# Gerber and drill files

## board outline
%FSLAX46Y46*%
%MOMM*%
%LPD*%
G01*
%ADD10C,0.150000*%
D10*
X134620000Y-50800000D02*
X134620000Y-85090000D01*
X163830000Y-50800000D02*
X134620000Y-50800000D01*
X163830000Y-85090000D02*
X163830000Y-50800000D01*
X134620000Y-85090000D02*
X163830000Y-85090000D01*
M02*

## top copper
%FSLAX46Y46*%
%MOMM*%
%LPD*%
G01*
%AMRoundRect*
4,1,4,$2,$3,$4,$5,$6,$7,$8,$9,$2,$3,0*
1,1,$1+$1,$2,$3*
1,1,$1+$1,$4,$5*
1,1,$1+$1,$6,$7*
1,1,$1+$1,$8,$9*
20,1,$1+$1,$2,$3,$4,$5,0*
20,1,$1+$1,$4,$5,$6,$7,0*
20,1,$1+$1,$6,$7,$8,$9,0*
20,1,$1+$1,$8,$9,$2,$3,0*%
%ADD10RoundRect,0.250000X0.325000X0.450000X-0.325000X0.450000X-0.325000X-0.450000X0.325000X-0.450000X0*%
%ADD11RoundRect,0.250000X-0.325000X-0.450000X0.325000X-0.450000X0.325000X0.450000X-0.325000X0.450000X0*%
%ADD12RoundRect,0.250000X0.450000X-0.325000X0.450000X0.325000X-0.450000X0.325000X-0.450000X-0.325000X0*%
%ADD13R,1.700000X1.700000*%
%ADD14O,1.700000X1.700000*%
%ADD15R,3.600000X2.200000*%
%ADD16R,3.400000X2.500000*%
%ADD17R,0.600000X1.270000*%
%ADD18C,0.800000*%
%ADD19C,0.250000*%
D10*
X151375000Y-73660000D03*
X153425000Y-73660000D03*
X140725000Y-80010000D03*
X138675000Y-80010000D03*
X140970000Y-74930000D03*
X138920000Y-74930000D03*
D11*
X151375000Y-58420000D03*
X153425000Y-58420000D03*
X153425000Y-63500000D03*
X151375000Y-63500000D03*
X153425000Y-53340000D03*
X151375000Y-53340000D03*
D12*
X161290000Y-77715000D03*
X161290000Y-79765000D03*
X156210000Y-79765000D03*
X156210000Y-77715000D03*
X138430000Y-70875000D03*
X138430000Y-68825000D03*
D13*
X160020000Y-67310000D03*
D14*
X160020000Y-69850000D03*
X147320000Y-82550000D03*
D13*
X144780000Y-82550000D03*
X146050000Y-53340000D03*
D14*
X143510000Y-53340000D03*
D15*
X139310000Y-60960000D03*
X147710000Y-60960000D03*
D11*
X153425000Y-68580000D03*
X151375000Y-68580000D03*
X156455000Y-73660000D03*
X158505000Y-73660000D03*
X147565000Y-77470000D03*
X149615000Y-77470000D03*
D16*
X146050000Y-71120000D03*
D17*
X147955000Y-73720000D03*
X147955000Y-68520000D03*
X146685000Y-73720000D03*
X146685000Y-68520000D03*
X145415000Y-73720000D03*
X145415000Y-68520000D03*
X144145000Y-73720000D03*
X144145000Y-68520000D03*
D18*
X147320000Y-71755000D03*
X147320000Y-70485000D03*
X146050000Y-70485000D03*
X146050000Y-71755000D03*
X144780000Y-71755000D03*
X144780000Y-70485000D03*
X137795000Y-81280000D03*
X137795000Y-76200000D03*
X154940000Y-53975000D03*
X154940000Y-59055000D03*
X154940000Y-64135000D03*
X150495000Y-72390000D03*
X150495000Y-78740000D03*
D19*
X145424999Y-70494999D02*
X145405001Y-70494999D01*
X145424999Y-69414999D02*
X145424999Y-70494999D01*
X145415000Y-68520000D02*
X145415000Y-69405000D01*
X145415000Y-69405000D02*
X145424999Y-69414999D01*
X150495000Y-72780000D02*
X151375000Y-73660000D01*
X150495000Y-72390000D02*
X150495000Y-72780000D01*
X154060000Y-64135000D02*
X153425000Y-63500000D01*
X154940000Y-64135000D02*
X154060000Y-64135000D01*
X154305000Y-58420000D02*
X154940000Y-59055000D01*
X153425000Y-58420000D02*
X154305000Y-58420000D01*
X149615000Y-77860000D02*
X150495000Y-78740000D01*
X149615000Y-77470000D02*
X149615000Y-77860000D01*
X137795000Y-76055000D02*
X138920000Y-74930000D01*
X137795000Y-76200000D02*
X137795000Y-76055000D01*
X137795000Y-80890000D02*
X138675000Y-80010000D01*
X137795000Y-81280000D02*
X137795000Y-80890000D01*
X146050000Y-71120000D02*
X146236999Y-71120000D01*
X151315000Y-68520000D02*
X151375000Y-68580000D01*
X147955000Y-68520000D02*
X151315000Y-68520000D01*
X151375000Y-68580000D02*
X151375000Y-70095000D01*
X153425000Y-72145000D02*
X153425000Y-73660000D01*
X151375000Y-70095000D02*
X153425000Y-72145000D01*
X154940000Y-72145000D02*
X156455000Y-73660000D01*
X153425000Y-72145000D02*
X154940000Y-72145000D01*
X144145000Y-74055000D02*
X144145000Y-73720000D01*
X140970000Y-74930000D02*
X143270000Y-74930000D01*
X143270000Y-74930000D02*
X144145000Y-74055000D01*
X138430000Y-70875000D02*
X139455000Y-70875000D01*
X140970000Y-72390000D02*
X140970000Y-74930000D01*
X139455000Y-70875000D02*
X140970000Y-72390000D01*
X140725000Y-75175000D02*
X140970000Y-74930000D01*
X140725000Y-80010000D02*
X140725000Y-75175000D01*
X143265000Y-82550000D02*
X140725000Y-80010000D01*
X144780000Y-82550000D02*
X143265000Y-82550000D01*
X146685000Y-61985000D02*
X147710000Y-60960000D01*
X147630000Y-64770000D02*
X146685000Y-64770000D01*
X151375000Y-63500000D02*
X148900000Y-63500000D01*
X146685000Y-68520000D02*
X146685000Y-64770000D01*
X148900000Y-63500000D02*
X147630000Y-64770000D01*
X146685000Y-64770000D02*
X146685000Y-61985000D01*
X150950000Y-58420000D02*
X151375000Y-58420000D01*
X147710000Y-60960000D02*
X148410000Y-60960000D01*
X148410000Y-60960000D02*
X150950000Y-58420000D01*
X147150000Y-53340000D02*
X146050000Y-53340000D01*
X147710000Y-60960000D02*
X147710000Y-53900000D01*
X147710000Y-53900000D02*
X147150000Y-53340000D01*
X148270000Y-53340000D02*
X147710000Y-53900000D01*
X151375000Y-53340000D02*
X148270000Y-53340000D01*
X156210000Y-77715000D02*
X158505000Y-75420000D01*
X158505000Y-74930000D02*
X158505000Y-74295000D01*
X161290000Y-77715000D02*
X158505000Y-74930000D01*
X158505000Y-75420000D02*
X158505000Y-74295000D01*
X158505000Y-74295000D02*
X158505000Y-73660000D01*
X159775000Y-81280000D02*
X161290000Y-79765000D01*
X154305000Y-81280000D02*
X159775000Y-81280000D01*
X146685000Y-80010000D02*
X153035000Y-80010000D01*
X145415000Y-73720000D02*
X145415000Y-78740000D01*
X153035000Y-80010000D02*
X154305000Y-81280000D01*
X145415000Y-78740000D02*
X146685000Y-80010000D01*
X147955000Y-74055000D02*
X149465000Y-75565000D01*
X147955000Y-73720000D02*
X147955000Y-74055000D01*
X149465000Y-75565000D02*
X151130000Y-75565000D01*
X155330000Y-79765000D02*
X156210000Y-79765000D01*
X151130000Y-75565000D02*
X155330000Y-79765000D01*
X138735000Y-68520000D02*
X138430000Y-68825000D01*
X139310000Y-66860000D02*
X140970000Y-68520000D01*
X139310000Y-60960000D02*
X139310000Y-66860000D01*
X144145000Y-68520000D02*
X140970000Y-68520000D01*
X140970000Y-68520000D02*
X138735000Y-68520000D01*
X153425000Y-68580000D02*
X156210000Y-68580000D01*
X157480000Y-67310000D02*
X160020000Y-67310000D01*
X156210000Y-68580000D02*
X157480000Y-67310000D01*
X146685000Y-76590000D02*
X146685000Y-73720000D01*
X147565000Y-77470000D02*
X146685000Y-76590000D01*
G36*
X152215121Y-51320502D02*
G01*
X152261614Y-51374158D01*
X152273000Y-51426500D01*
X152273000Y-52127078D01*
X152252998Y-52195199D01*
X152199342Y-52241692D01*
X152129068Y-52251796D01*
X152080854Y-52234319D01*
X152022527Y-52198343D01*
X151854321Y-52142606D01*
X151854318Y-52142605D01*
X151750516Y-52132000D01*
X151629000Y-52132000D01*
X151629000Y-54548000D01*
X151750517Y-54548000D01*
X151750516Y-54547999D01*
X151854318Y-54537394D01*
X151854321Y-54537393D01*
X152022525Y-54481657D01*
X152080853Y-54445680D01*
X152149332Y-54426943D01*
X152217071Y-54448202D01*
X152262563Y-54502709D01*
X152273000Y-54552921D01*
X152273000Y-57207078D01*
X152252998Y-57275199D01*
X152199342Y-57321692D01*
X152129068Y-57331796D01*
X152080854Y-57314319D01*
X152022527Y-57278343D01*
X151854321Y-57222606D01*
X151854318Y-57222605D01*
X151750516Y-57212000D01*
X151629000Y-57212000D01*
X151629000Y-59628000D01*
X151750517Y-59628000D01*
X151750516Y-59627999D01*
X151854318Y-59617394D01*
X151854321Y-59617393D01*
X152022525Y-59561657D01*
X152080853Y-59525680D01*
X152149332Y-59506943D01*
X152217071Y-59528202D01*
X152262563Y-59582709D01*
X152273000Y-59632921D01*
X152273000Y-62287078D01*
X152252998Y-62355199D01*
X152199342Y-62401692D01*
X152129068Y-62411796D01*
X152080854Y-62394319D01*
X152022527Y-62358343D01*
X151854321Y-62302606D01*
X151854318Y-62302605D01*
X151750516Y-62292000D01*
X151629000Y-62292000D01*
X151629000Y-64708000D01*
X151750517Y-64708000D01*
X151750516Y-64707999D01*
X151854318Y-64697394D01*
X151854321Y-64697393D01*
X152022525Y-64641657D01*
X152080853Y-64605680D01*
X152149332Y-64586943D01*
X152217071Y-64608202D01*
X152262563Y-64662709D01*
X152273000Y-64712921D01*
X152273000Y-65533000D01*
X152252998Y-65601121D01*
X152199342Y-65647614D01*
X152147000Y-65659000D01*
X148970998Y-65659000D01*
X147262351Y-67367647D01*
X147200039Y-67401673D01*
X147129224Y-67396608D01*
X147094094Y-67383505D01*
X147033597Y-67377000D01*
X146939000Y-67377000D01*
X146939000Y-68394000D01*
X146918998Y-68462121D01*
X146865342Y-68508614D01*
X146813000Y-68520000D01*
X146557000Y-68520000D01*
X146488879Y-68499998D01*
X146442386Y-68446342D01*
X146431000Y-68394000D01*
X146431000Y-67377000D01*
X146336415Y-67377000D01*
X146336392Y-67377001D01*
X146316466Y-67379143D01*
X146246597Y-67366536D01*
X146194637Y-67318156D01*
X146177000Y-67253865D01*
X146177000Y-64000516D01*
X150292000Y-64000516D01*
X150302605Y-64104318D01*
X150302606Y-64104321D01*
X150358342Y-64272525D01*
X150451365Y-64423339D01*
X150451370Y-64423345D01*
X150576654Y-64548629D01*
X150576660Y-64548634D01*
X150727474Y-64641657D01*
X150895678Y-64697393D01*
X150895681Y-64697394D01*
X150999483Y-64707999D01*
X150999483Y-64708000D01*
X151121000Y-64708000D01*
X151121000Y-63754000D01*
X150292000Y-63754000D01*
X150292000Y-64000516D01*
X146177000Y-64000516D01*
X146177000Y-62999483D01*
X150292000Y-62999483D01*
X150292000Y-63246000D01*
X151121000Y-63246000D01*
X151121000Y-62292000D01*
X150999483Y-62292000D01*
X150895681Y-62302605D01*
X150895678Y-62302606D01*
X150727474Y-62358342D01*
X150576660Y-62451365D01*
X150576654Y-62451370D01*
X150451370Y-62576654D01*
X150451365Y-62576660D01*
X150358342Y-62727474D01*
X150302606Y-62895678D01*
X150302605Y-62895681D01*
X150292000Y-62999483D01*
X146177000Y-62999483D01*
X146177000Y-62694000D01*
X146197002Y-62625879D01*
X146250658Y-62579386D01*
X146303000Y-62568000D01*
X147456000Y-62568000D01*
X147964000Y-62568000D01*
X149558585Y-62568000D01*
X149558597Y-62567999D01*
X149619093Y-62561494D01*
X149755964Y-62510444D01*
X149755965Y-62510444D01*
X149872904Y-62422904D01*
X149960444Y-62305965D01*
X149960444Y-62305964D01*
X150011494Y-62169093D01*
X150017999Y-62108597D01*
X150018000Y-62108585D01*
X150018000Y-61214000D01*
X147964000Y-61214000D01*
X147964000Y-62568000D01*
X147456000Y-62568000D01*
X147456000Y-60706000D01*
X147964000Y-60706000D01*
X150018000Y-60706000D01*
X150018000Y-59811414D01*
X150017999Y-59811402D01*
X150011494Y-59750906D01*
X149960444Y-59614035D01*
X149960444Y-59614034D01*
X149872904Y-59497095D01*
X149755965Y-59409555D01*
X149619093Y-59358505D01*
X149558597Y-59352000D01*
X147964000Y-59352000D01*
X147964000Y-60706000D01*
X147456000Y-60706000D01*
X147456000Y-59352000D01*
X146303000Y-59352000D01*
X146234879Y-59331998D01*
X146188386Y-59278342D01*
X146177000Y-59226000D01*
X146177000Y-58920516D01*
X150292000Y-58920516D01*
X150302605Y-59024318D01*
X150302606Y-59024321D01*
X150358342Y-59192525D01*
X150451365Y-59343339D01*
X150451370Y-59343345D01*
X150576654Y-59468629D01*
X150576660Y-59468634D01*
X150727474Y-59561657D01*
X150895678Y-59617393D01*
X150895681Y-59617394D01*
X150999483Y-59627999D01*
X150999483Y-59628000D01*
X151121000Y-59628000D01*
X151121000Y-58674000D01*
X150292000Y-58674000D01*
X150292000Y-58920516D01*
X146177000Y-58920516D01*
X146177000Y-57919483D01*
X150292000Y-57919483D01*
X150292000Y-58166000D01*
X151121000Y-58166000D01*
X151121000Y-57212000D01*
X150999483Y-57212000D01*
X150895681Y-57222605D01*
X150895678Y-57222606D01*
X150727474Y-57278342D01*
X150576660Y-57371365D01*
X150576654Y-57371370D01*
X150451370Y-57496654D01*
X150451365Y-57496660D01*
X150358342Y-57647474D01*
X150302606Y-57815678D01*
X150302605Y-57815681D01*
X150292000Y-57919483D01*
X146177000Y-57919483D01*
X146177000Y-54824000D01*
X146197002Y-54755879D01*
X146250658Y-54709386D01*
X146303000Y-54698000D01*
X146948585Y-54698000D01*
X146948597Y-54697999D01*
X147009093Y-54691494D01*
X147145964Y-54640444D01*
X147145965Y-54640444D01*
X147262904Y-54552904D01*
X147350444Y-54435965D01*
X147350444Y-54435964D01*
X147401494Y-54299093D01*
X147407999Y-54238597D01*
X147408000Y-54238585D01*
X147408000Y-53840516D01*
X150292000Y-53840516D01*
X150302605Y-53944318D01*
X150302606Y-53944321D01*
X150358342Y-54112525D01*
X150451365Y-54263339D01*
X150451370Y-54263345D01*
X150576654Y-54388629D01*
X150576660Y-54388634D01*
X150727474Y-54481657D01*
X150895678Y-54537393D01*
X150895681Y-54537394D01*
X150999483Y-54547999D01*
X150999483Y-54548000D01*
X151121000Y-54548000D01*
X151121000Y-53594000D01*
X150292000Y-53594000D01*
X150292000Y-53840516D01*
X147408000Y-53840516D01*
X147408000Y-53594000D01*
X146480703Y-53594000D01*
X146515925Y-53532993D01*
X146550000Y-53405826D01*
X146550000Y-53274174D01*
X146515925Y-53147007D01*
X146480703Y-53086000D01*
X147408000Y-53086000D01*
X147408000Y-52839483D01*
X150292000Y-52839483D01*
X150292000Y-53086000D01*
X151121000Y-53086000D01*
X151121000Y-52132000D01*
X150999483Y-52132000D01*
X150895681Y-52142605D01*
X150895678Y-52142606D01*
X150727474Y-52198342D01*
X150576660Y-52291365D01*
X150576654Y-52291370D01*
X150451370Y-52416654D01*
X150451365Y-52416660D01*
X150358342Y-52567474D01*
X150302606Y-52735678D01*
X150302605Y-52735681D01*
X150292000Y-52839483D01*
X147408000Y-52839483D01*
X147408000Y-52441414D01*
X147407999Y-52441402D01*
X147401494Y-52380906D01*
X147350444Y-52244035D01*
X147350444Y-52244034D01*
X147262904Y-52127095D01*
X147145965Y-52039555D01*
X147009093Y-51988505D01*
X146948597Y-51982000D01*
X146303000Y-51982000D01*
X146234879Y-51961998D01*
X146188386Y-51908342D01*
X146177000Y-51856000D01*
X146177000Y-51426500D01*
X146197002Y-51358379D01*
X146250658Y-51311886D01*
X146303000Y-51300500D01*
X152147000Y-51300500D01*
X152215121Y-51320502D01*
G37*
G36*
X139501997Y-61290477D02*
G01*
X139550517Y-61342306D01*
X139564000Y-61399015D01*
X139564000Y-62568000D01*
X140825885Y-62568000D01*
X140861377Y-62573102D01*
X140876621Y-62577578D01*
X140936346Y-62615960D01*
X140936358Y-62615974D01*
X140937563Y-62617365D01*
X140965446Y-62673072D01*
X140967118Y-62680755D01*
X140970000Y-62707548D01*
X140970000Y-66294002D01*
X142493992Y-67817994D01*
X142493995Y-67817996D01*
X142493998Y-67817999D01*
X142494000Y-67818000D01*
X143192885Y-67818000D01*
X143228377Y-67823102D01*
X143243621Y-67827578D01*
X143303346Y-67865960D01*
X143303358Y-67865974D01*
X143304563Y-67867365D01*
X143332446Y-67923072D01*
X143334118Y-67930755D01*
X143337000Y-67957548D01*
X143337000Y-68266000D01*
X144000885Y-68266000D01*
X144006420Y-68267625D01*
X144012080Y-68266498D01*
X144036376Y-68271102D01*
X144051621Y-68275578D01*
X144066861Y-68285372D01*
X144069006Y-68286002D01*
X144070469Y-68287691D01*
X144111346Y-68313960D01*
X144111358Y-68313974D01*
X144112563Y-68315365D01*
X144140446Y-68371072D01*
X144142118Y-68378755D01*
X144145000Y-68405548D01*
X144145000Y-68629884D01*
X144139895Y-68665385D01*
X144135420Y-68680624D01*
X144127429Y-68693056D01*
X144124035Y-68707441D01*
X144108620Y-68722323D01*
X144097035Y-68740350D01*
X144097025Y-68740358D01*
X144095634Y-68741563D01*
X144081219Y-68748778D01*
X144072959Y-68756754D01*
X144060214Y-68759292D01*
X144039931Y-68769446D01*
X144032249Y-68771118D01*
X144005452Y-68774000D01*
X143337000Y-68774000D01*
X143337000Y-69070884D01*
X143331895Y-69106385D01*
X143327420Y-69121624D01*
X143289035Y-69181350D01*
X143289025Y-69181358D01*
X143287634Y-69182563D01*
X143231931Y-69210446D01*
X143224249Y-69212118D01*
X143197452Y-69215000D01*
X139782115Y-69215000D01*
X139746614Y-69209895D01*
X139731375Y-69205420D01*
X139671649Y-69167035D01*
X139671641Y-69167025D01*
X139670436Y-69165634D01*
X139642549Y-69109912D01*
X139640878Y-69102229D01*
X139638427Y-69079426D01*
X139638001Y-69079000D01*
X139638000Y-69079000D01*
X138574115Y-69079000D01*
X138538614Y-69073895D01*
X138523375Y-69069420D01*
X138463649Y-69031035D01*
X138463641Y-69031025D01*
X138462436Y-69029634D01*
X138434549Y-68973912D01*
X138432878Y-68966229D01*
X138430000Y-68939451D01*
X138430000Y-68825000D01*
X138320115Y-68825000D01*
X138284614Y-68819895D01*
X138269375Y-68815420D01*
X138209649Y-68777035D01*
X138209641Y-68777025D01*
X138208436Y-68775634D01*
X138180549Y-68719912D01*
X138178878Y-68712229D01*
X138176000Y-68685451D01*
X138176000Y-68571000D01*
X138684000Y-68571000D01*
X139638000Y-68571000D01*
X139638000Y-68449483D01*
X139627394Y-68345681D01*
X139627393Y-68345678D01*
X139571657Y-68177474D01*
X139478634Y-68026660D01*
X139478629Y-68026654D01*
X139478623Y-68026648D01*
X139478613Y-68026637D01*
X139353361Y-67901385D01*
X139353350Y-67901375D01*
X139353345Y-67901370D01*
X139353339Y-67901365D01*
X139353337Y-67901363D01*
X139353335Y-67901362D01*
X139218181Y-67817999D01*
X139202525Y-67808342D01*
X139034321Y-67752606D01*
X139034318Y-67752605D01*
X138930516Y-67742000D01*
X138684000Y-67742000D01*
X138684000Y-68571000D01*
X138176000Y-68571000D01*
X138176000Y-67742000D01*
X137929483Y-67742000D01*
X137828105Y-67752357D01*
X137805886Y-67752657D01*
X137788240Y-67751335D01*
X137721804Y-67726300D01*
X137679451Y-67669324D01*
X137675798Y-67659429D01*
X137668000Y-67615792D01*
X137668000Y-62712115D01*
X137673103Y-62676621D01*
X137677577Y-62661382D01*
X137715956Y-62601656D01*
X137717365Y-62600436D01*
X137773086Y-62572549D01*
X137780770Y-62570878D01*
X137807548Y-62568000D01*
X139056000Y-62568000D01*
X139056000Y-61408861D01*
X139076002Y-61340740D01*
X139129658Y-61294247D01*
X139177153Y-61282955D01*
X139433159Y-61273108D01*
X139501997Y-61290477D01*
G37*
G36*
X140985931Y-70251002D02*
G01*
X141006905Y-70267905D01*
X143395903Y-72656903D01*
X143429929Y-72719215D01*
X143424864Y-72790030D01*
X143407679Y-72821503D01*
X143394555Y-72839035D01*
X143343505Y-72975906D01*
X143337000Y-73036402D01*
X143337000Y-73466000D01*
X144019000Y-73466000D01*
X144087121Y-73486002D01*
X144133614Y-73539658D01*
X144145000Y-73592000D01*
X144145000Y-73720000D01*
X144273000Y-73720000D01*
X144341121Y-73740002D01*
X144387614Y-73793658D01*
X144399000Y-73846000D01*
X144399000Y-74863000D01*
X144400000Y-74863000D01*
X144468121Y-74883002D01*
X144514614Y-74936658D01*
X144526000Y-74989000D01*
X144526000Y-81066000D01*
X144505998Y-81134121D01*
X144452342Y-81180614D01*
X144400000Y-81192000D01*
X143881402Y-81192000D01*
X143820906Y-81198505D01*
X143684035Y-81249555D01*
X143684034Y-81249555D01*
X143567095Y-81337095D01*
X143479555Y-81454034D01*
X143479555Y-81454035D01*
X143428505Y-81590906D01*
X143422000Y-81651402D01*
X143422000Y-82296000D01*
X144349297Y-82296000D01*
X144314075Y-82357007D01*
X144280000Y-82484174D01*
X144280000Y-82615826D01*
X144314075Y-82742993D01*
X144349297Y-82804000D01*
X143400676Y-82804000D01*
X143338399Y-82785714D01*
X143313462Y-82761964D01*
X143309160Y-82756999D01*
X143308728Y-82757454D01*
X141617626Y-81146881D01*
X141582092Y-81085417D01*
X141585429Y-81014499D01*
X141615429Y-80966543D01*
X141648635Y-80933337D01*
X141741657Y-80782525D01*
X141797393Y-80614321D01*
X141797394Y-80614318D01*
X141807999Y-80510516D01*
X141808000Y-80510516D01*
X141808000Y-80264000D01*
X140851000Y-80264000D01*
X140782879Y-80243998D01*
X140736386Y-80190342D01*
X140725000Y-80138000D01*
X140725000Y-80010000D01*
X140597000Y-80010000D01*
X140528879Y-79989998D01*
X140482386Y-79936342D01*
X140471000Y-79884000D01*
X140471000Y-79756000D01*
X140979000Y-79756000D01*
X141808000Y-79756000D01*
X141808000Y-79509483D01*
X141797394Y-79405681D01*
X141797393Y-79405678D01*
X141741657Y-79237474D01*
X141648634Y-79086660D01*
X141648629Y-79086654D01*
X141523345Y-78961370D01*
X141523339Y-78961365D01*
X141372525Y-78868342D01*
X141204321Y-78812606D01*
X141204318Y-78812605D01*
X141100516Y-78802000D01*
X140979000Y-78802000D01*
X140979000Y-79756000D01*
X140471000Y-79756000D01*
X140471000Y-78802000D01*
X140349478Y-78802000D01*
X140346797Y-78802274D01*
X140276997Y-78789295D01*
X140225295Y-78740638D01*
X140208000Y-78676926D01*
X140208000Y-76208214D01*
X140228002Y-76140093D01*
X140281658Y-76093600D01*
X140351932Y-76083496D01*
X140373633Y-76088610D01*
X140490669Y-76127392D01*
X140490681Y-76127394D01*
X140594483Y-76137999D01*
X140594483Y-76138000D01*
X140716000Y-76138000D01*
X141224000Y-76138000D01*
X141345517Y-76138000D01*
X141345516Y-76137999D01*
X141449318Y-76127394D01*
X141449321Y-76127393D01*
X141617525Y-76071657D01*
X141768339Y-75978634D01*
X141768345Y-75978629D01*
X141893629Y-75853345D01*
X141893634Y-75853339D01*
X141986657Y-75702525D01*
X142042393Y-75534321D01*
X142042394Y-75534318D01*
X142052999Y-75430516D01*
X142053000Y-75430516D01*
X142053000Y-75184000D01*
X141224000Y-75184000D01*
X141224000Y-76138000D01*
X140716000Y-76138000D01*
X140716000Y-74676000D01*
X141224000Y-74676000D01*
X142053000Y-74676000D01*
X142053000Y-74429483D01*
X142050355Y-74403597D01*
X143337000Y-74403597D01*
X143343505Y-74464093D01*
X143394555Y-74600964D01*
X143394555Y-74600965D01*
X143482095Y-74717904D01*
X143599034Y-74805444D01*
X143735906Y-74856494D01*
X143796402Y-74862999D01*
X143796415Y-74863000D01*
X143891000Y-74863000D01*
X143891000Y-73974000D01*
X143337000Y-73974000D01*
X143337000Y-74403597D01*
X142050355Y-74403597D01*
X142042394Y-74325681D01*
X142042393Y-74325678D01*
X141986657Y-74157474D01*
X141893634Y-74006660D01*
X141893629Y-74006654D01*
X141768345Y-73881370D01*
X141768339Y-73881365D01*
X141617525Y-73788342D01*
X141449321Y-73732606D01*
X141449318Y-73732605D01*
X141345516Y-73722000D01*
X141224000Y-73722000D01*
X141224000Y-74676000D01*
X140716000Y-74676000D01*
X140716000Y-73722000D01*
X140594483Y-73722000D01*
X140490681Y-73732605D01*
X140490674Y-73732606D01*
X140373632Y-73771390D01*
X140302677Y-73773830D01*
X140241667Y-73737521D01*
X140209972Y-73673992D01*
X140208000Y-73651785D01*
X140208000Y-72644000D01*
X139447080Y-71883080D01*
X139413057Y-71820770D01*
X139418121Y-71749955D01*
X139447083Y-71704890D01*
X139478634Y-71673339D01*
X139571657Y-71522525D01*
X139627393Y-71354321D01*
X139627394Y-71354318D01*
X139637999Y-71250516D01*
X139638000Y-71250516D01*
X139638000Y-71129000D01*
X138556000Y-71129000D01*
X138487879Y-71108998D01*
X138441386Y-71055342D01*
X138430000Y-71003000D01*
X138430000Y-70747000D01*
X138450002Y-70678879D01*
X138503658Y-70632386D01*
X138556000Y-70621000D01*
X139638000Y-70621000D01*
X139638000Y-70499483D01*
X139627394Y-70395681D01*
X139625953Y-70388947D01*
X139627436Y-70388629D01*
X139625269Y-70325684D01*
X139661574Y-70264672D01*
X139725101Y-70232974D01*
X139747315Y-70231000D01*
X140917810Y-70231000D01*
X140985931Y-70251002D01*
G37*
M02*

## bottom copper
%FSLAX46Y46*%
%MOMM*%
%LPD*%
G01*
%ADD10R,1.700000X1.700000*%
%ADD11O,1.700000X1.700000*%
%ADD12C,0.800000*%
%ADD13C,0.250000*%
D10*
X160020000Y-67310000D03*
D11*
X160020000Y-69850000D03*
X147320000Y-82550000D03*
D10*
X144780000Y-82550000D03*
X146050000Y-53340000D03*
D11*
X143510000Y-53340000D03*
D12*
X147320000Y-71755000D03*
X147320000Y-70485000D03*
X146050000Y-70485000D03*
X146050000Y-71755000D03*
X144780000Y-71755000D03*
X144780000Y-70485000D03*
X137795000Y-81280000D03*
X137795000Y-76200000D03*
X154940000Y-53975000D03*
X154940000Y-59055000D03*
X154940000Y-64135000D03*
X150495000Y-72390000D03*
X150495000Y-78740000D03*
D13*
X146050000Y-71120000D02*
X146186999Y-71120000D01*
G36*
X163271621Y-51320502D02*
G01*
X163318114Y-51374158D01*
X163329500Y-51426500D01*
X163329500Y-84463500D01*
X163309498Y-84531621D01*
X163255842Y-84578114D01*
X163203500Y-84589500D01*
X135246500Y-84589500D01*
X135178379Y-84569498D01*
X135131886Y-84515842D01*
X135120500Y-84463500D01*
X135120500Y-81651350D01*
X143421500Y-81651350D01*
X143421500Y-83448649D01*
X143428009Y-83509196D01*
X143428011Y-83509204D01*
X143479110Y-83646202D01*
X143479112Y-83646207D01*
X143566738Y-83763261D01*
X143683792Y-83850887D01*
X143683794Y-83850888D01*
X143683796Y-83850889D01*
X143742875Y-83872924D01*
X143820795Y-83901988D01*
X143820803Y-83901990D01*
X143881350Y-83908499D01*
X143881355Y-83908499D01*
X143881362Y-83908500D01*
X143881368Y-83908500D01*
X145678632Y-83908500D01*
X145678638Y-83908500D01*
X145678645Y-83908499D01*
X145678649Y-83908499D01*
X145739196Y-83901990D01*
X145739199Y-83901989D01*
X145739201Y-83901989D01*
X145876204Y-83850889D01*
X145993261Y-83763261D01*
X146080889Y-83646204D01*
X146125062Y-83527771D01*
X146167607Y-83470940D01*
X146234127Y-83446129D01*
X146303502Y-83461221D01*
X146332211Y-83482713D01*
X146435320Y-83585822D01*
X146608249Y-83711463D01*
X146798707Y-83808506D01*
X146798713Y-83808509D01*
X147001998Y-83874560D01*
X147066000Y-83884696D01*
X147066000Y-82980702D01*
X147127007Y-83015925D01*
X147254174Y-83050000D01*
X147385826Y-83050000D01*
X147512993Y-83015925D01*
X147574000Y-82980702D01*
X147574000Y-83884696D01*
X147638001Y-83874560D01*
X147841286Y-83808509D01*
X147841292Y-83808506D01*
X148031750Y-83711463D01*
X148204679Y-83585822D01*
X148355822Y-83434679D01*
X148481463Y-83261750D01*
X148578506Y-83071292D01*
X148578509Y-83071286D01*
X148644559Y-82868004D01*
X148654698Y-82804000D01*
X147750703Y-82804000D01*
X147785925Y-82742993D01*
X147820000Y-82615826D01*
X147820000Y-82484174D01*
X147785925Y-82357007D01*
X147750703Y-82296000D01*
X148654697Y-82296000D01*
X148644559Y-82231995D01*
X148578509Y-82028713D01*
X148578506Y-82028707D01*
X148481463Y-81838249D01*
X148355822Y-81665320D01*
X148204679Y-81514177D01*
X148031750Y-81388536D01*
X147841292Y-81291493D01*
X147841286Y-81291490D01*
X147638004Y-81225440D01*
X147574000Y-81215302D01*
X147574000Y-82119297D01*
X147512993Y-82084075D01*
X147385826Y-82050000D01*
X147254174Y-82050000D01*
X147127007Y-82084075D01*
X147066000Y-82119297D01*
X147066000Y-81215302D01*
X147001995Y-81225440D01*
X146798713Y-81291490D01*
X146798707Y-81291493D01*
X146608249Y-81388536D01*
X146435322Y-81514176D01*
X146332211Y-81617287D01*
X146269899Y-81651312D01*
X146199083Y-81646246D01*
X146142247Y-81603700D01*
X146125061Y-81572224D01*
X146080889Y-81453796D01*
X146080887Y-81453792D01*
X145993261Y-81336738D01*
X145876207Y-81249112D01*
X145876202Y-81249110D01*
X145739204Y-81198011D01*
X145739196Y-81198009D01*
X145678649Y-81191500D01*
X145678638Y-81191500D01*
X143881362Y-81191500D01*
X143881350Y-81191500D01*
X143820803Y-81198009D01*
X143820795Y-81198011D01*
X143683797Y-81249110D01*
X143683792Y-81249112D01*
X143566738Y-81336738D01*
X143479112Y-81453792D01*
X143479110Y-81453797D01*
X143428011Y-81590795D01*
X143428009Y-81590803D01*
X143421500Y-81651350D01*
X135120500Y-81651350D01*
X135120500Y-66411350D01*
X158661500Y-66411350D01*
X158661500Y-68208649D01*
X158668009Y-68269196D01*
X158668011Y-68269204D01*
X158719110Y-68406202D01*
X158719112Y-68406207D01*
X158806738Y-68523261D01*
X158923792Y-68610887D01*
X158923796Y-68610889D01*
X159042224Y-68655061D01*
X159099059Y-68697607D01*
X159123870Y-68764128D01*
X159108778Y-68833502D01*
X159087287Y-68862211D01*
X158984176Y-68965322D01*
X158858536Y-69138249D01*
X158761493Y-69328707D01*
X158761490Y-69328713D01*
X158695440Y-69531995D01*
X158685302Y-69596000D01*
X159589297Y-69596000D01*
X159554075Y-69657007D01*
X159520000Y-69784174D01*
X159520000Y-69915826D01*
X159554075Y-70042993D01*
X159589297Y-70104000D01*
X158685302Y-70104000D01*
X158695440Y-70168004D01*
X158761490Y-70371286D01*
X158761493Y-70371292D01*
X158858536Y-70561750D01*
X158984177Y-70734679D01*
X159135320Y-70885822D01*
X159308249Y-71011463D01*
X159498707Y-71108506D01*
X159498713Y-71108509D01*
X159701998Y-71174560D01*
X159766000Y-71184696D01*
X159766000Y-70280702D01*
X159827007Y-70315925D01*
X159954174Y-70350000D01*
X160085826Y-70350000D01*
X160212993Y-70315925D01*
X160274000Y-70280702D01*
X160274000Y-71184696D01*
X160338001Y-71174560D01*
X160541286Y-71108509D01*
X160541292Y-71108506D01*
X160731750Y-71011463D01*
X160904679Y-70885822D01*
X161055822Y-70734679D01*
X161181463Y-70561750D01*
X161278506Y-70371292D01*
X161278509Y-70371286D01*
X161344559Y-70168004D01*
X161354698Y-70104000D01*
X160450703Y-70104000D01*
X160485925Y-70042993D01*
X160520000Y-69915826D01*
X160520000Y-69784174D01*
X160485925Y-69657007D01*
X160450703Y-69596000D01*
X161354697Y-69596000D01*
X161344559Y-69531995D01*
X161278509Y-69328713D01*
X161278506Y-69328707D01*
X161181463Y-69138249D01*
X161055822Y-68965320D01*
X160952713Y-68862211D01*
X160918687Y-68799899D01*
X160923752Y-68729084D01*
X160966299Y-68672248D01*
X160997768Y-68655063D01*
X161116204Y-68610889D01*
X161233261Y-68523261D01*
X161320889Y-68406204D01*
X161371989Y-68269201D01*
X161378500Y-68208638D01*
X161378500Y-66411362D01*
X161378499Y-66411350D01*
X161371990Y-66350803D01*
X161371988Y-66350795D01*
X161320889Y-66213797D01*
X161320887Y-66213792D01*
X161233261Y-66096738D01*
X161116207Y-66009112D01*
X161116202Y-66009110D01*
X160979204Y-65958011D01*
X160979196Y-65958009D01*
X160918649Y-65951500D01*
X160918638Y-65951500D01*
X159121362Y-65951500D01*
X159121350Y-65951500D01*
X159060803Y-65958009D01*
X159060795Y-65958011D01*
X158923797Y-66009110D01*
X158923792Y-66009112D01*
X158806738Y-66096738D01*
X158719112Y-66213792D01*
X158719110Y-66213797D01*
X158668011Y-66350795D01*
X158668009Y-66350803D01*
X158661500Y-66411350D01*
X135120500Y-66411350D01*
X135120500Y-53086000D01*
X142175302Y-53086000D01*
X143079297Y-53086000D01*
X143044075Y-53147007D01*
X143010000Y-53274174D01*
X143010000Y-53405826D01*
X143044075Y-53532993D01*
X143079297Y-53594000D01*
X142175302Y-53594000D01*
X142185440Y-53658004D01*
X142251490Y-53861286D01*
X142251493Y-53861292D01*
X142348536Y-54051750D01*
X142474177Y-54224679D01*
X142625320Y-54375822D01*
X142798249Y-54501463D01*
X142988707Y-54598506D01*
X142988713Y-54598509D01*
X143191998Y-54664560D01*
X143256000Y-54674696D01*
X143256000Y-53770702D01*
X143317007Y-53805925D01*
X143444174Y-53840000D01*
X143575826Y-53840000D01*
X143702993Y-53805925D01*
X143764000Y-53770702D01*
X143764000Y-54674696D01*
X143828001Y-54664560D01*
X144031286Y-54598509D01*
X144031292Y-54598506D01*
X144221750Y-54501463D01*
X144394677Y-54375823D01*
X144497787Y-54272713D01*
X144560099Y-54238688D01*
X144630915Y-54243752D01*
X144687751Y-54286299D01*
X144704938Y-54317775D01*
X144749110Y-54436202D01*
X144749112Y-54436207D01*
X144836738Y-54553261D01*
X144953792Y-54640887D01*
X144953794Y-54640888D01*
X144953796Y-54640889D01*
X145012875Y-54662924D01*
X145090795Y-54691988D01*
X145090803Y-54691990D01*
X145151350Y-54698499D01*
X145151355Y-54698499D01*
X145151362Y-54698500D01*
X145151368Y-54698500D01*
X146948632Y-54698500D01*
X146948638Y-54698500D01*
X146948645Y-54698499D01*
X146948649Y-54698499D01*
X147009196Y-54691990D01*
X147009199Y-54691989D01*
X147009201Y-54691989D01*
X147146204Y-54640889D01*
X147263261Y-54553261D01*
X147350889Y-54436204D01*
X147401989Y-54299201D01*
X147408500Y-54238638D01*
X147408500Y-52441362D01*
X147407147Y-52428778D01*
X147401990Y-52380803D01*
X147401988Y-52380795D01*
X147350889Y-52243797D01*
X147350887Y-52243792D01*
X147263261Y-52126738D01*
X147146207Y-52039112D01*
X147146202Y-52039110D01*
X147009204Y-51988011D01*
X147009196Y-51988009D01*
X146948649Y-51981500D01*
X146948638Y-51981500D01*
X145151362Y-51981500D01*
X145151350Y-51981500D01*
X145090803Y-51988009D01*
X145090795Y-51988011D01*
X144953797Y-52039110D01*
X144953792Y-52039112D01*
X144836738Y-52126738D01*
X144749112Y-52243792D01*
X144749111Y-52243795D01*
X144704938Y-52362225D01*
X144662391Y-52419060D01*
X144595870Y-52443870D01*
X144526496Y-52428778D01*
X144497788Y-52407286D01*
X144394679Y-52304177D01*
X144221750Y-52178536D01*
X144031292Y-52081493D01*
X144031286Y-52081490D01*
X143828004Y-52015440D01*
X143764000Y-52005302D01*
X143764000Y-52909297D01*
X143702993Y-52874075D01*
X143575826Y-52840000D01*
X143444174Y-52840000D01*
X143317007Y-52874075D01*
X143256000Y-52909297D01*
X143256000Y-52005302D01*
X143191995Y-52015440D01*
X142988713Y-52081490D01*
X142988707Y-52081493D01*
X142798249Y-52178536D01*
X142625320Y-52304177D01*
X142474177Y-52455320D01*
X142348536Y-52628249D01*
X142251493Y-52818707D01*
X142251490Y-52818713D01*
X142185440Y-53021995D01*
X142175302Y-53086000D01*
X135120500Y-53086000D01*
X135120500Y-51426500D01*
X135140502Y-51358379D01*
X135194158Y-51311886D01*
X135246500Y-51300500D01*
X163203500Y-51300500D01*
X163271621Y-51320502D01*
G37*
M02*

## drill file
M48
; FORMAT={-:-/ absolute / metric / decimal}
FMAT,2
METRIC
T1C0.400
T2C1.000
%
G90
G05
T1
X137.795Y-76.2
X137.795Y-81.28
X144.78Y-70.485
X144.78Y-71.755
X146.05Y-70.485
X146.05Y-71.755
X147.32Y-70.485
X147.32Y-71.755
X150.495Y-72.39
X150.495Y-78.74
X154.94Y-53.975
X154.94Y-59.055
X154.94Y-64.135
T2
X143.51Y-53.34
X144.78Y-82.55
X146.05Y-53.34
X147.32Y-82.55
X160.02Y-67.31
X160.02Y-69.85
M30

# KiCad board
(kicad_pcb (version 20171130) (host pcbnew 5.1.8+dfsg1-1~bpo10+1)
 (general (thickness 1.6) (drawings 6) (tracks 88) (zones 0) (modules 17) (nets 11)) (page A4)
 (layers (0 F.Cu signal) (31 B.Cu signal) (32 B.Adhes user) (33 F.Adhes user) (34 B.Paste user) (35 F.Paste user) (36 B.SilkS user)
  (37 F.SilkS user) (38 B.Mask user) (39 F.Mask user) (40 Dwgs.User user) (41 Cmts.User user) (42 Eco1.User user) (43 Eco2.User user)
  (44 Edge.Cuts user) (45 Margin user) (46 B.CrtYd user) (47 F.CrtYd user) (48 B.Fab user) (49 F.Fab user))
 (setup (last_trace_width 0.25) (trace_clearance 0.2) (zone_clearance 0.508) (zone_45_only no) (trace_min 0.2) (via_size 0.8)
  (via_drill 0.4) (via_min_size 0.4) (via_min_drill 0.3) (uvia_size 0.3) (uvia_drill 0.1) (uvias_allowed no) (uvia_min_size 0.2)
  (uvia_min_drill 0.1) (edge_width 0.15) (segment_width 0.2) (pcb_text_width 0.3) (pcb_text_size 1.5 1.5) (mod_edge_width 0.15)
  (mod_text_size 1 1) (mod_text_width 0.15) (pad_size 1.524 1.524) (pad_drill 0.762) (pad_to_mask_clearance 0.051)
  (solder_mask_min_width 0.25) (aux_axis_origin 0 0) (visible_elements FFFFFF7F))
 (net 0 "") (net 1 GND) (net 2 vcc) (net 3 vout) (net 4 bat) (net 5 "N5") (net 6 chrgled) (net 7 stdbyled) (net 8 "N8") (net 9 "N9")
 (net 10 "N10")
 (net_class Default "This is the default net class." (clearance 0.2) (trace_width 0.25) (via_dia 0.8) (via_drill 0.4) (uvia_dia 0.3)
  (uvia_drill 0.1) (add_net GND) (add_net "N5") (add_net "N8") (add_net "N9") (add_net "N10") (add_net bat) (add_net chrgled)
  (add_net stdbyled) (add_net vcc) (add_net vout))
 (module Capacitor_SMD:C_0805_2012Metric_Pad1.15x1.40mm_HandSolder (layer F.Cu) (at 152.4 73.66 180)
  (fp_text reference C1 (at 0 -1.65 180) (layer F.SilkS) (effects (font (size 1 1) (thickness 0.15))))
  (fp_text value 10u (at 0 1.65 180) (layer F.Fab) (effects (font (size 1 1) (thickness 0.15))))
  (pad 2 smd roundrect (at 1.025 0 180) (size 1.15 1.4) (layers F.Cu F.Paste F.Mask) (roundrect_rratio 0.217391) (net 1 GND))
  (pad 1 smd roundrect (at -1.025 0 180) (size 1.15 1.4) (layers F.Cu F.Paste F.Mask) (roundrect_rratio 0.217391) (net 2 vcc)))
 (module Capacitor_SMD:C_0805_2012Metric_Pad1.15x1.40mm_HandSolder (layer F.Cu) (at 139.7 80.01 180)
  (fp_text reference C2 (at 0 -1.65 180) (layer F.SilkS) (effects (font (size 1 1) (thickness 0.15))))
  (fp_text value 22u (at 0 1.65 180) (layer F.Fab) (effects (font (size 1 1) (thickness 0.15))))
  (pad 1 smd roundrect (at -1.025 0 180) (size 1.15 1.4) (layers F.Cu F.Paste F.Mask) (roundrect_rratio 0.217391) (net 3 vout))
  (pad 2 smd roundrect (at 1.025 0 180) (size 1.15 1.4) (layers F.Cu F.Paste F.Mask) (roundrect_rratio 0.217391) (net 1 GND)))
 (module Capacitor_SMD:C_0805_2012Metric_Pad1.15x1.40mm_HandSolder (layer F.Cu) (at 139.945 74.93 180)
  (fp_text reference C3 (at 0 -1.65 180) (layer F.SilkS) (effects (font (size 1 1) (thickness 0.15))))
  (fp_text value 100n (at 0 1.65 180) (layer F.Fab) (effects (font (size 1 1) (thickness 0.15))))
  (pad 1 smd roundrect (at -1.025 0 180) (size 1.15 1.4) (layers F.Cu F.Paste F.Mask) (roundrect_rratio 0.217391) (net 3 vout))
  (pad 2 smd roundrect (at 1.025 0 180) (size 1.15 1.4) (layers F.Cu F.Paste F.Mask) (roundrect_rratio 0.217391) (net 1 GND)))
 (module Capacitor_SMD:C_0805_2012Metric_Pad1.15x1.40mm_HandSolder (layer F.Cu) (at 152.4 58.42)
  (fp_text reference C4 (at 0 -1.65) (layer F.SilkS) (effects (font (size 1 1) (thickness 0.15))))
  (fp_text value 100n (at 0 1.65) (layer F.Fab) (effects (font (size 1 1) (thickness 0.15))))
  (pad 1 smd roundrect (at -1.025 0) (size 1.15 1.4) (layers F.Cu F.Paste F.Mask) (roundrect_rratio 0.217391) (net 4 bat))
  (pad 2 smd roundrect (at 1.025 0) (size 1.15 1.4) (layers F.Cu F.Paste F.Mask) (roundrect_rratio 0.217391) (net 1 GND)))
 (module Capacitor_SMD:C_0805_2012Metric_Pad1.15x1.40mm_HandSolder (layer F.Cu) (at 152.4 63.5)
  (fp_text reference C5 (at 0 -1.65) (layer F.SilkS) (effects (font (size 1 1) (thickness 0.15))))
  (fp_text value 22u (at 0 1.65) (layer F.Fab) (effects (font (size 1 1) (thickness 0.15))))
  (pad 2 smd roundrect (at 1.025 0) (size 1.15 1.4) (layers F.Cu F.Paste F.Mask) (roundrect_rratio 0.217391) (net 1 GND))
  (pad 1 smd roundrect (at -1.025 0) (size 1.15 1.4) (layers F.Cu F.Paste F.Mask) (roundrect_rratio 0.217391) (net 4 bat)))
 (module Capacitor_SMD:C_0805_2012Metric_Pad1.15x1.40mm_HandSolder (layer F.Cu) (at 152.4 53.34)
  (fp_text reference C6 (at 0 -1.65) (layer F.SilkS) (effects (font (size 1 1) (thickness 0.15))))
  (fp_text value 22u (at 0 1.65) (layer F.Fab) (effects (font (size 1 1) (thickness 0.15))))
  (pad 2 smd roundrect (at 1.025 0) (size 1.15 1.4) (layers F.Cu F.Paste F.Mask) (roundrect_rratio 0.217391) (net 1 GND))
  (pad 1 smd roundrect (at -1.025 0) (size 1.15 1.4) (layers F.Cu F.Paste F.Mask) (roundrect_rratio 0.217391) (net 4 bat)))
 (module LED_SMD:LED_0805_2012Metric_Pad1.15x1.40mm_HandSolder (layer F.Cu) (at 161.29 78.74 90)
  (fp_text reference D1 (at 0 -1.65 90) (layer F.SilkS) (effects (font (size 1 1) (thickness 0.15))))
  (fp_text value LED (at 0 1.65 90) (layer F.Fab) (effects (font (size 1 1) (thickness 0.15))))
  (pad 2 smd roundrect (at 1.025 0 90) (size 1.15 1.4) (layers F.Cu F.Paste F.Mask) (roundrect_rratio 0.217391) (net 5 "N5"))
  (pad 1 smd roundrect (at -1.025 0 90) (size 1.15 1.4) (layers F.Cu F.Paste F.Mask) (roundrect_rratio 0.217391) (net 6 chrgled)))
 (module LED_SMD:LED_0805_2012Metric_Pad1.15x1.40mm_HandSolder (layer F.Cu) (at 156.21 78.74 90)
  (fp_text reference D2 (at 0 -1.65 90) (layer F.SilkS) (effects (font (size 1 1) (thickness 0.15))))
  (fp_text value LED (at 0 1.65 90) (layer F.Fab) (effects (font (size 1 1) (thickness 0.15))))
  (pad 1 smd roundrect (at -1.025 0 90) (size 1.15 1.4) (layers F.Cu F.Paste F.Mask) (roundrect_rratio 0.217391) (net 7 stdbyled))
  (pad 2 smd roundrect (at 1.025 0 90) (size 1.15 1.4) (layers F.Cu F.Paste F.Mask) (roundrect_rratio 0.217391) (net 5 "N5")))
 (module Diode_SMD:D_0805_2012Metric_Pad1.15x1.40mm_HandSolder (layer F.Cu) (at 138.43 69.85 90)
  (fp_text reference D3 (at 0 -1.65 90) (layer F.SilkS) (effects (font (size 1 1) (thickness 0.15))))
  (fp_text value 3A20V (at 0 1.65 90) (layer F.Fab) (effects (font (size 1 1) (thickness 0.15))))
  (pad 1 smd roundrect (at -1.025 0 90) (size 1.15 1.4) (layers F.Cu F.Paste F.Mask) (roundrect_rratio 0.217391) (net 3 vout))
  (pad 2 smd roundrect (at 1.025 0 90) (size 1.15 1.4) (layers F.Cu F.Paste F.Mask) (roundrect_rratio 0.217391) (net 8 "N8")))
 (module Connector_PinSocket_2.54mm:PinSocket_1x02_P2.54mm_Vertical (layer F.Cu) (at 160.02 67.31)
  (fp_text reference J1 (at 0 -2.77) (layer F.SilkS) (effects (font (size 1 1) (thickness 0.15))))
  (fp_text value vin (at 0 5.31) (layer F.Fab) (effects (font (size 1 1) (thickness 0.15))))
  (pad 1 thru_hole rect (at 0 0) (size 1.7 1.7) (drill 1) (layers *.Cu *.Mask) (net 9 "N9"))
  (pad 2 thru_hole oval (at 0 2.54) (size 1.7 1.7) (drill 1) (layers *.Cu *.Mask) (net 1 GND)))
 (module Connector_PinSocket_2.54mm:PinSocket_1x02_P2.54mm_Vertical (layer F.Cu) (at 144.78 82.55 90)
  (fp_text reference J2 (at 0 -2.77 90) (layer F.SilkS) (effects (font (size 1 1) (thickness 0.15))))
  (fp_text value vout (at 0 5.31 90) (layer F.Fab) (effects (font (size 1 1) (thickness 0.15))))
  (pad 2 thru_hole oval (at 0 2.54 90) (size 1.7 1.7) (drill 1) (layers *.Cu *.Mask) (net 1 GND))
  (pad 1 thru_hole rect (at 0 0 90) (size 1.7 1.7) (drill 1) (layers *.Cu *.Mask) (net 3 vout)))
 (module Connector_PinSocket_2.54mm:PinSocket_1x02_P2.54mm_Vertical (layer F.Cu) (at 146.05 53.34 270)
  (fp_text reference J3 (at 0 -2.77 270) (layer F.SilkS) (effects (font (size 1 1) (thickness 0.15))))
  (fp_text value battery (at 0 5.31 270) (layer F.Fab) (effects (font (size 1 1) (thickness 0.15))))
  (pad 1 thru_hole rect (at 0 0 270) (size 1.7 1.7) (drill 1) (layers *.Cu *.Mask) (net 4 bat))
  (pad 2 thru_hole oval (at 0 2.54 270) (size 1.7 1.7) (drill 1) (layers *.Cu *.Mask) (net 1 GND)))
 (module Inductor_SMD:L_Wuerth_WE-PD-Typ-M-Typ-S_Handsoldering (layer F.Cu) (at 143.51 60.96)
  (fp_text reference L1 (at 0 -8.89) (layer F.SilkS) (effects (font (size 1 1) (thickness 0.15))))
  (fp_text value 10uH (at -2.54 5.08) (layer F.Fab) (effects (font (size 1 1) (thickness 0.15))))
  (pad 1 smd rect (at -4.2 0) (size 3.6 2.2) (layers F.Cu F.Paste F.Mask) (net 8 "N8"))
  (pad 2 smd rect (at 4.2 0) (size 3.6 2.2) (layers F.Cu F.Paste F.Mask) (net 4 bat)))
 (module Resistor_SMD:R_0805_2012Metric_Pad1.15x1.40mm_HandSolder (layer F.Cu) (at 152.4 68.58)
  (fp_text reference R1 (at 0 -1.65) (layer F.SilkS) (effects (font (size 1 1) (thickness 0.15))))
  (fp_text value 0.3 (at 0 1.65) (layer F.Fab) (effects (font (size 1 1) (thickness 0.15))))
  (pad 2 smd roundrect (at 1.025 0) (size 1.15 1.4) (layers F.Cu F.Paste F.Mask) (roundrect_rratio 0.217391) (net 9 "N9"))
  (pad 1 smd roundrect (at -1.025 0) (size 1.15 1.4) (layers F.Cu F.Paste F.Mask) (roundrect_rratio 0.217391) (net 2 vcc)))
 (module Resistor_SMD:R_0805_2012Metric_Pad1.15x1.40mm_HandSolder (layer F.Cu) (at 157.48 73.66)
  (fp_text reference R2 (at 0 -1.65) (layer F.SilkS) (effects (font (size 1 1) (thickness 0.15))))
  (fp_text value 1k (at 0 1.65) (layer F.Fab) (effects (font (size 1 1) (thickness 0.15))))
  (pad 1 smd roundrect (at -1.025 0) (size 1.15 1.4) (layers F.Cu F.Paste F.Mask) (roundrect_rratio 0.217391) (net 2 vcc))
  (pad 2 smd roundrect (at 1.025 0) (size 1.15 1.4) (layers F.Cu F.Paste F.Mask) (roundrect_rratio 0.217391) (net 5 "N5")))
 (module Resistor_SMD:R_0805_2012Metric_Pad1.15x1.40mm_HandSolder (layer F.Cu) (at 148.59 77.47)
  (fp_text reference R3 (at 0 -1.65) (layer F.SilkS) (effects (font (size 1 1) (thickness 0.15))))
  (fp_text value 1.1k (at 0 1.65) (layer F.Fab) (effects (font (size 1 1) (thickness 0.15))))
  (pad 1 smd roundrect (at -1.025 0) (size 1.15 1.4) (layers F.Cu F.Paste F.Mask) (roundrect_rratio 0.217391) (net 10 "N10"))
  (pad 2 smd roundrect (at 1.025 0) (size 1.15 1.4) (layers F.Cu F.Paste F.Mask) (roundrect_rratio 0.217391) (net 1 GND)))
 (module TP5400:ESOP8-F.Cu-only (layer F.Cu) (at 146.05 71.12)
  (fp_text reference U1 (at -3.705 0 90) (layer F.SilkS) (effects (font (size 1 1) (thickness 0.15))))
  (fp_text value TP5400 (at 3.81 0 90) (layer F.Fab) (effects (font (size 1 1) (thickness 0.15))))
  (pad 9 smd rect (at 0 0) (size 3.4 2.5) (layers F.Cu F.Paste F.Mask) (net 1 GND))
  (pad 4 smd rect (at 1.905 2.6) (size 0.6 1.27) (layers F.Cu F.Paste F.Mask) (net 7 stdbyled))
  (pad 5 smd rect (at 1.905 -2.6) (size 0.6 1.27) (layers F.Cu F.Paste F.Mask) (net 2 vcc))
  (pad 3 smd rect (at 0.635 2.6) (size 0.6 1.27) (layers F.Cu F.Paste F.Mask) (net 10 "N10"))
  (pad 6 smd rect (at 0.635 -2.6) (size 0.6 1.27) (layers F.Cu F.Paste F.Mask) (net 4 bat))
  (pad 2 smd rect (at -0.635 2.6) (size 0.6 1.27) (layers F.Cu F.Paste F.Mask) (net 6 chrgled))
  (pad 7 smd rect (at -0.635 -2.6) (size 0.6 1.27) (layers F.Cu F.Paste F.Mask) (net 1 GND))
  (pad 1 smd rect (at -1.905 2.6) (size 0.6 1.27) (layers F.Cu F.Paste F.Mask) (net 3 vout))
  (pad 8 smd rect (at -1.905 -2.6) (size 0.6 1.27) (layers F.Cu F.Paste F.Mask) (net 8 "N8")))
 (gr_line (start 134.62 50.8) (end 134.62 85.09) (layer Edge.Cuts) (width 0.15))
 (gr_line (start 163.83 50.8) (end 134.62 50.8) (layer Edge.Cuts) (width 0.15))
 (gr_line (start 163.83 85.09) (end 163.83 50.8) (layer Edge.Cuts) (width 0.15))
 (gr_line (start 134.62 85.09) (end 163.83 85.09) (layer Edge.Cuts) (width 0.15))
 (via (at 147.32 71.755) (size 0.8) (drill 0.4) (layers F.Cu B.Cu) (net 1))
 (via (at 147.32 70.485) (size 0.8) (drill 0.4) (layers F.Cu B.Cu) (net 1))
 (via (at 146.05 70.485) (size 0.8) (drill 0.4) (layers F.Cu B.Cu) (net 1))
 (via (at 146.05 71.755) (size 0.8) (drill 0.4) (layers F.Cu B.Cu) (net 1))
 (via (at 144.78 71.755) (size 0.8) (drill 0.4) (layers F.Cu B.Cu) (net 1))
 (via (at 144.78 70.485) (size 0.8) (drill 0.4) (layers F.Cu B.Cu) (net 1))
 (segment (start 145.424999 70.494999) (end 145.405001 70.494999) (width 0.25) (layer F.Cu) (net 1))
 (segment (start 145.424999 69.414999) (end 145.424999 70.494999) (width 0.25) (layer F.Cu) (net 1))
 (segment (start 145.415 68.52) (end 145.415 69.405) (width 0.25) (layer F.Cu) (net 1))
 (segment (start 145.415 69.405) (end 145.424999 69.414999) (width 0.25) (layer F.Cu) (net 1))
 (via (at 137.795 81.28) (size 0.8) (drill 0.4) (layers F.Cu B.Cu) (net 1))
 (via (at 137.795 76.2) (size 0.8) (drill 0.4) (layers F.Cu B.Cu) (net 1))
 (via (at 154.94 53.975) (size 0.8) (drill 0.4) (layers F.Cu B.Cu) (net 1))
 (via (at 154.94 59.055) (size 0.8) (drill 0.4) (layers F.Cu B.Cu) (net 1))
 (via (at 154.94 64.135) (size 0.8) (drill 0.4) (layers F.Cu B.Cu) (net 1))
 (via (at 150.495 72.39) (size 0.8) (drill 0.4) (layers F.Cu B.Cu) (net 1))
 (via (at 150.495 78.74) (size 0.8) (drill 0.4) (layers F.Cu B.Cu) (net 1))
 (segment (start 150.495 72.78) (end 151.375 73.66) (width 0.25) (layer F.Cu) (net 1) (status 20))
 (segment (start 150.495 72.39) (end 150.495 72.78) (width 0.25) (layer F.Cu) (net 1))
 (segment (start 154.06 64.135) (end 153.425 63.5) (width 0.25) (layer F.Cu) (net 1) (status 20))
 (segment (start 154.94 64.135) (end 154.06 64.135) (width 0.25) (layer F.Cu) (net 1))
 (segment (start 154.305 58.42) (end 154.94 59.055) (width 0.25) (layer F.Cu) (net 1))
 (segment (start 153.425 58.42) (end 154.305 58.42) (width 0.25) (layer F.Cu) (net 1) (status 10))
 (segment (start 149.615 77.86) (end 150.495 78.74) (width 0.25) (layer F.Cu) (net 1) (status 10))
 (segment (start 149.615 77.47) (end 149.615 77.86) (width 0.25) (layer F.Cu) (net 1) (status 30))
 (segment (start 137.795 76.055) (end 138.92 74.93) (width 0.25) (layer F.Cu) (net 1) (status 20))
 (segment (start 137.795 76.2) (end 137.795 76.055) (width 0.25) (layer F.Cu) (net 1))
 (segment (start 137.795 80.89) (end 138.675 80.01) (width 0.25) (layer F.Cu) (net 1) (status 20))
 (segment (start 137.795 81.28) (end 137.795 80.89) (width 0.25) (layer F.Cu) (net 1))
 (segment (start 146.05 71.12) (end 146.186999 71.12) (width 0.25) (layer B.Cu) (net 1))
 (segment (start 146.05 71.12) (end 146.236999 71.12) (width 0.25) (layer F.Cu) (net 1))
 (segment (start 151.315 68.52) (end 151.375 68.58) (width 0.25) (layer F.Cu) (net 2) (status 30))
 (segment (start 147.955 68.52) (end 151.315 68.52) (width 0.25) (layer F.Cu) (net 2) (status 20))
 (segment (start 151.375 68.58) (end 151.375 70.095) (width 0.25) (layer F.Cu) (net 2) (status 10))
 (segment (start 153.425 72.145) (end 153.425 73.66) (width 0.25) (layer F.Cu) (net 2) (status 20))
 (segment (start 151.375 70.095) (end 153.425 72.145) (width 0.25) (layer F.Cu) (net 2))
 (segment (start 154.94 72.145) (end 156.455 73.66) (width 0.25) (layer F.Cu) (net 2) (status 20))
 (segment (start 153.425 72.145) (end 154.94 72.145) (width 0.25) (layer F.Cu) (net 2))
 (segment (start 144.145 74.055) (end 144.145 73.72) (width 0.25) (layer F.Cu) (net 3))
 (segment (start 140.97 74.93) (end 143.27 74.93) (width 0.25) (layer F.Cu) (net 3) (status 10))
 (segment (start 143.27 74.93) (end 144.145 74.055) (width 0.25) (layer F.Cu) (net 3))
 (segment (start 138.43 70.875) (end 139.455 70.875) (width 0.25) (layer F.Cu) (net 3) (status 10))
 (segment (start 140.97 72.39) (end 140.97 74.93) (width 0.25) (layer F.Cu) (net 3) (status 20))
 (segment (start 139.455 70.875) (end 140.97 72.39) (width 0.25) (layer F.Cu) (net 3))
 (segment (start 140.725 75.175) (end 140.97 74.93) (width 0.25) (layer F.Cu) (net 3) (status 30))
 (segment (start 140.725 80.01) (end 140.725 75.175) (width 0.25) (layer F.Cu) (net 3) (status 30))
 (segment (start 143.265 82.55) (end 140.725 80.01) (width 0.25) (layer F.Cu) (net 3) (status 20))
 (segment (start 144.78 82.55) (end 143.265 82.55) (width 0.25) (layer F.Cu) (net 3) (status 10))
 (segment (start 146.685 61.985) (end 147.71 60.96) (width 0.25) (layer F.Cu) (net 4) (status 30))
 (segment (start 147.63 64.77) (end 146.685 64.77) (width 0.25) (layer F.Cu) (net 4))
 (segment (start 151.375 63.5) (end 148.9 63.5) (width 0.25) (layer F.Cu) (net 4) (status 10))
 (segment (start 146.685 68.52) (end 146.685 64.77) (width 0.25) (layer F.Cu) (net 4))
 (segment (start 148.9 63.5) (end 147.63 64.77) (width 0.25) (layer F.Cu) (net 4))
 (segment (start 146.685 64.77) (end 146.685 61.985) (width 0.25) (layer F.Cu) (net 4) (status 20))
 (segment (start 150.95 58.42) (end 151.375 58.42) (width 0.25) (layer F.Cu) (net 4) (status 30))
 (segment (start 147.71 60.96) (end 148.41 60.96) (width 0.25) (layer F.Cu) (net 4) (status 30))
 (segment (start 148.41 60.96) (end 150.95 58.42) (width 0.25) (layer F.Cu) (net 4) (status 30))
 (segment (start 147.15 53.34) (end 146.05 53.34) (width 0.25) (layer F.Cu) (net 4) (status 20))
 (segment (start 147.71 60.96) (end 147.71 53.9) (width 0.25) (layer F.Cu) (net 4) (status 10))
 (segment (start 147.71 53.9) (end 147.15 53.34) (width 0.25) (layer F.Cu) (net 4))
 (segment (start 148.27 53.34) (end 147.71 53.9) (width 0.25) (layer F.Cu) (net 4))
 (segment (start 151.375 53.34) (end 148.27 53.34) (width 0.25) (layer F.Cu) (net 4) (status 10))
 (segment (start 156.21 77.715) (end 158.505 75.42) (width 0.25) (layer F.Cu) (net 5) (status 10))
 (segment (start 158.505 74.93) (end 158.505 74.295) (width 0.25) (layer F.Cu) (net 5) (status 20))
 (segment (start 161.29 77.715) (end 158.505 74.93) (width 0.25) (layer F.Cu) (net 5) (status 10))
 (segment (start 158.505 75.42) (end 158.505 74.295) (width 0.25) (layer F.Cu) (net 5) (status 20))
 (segment (start 158.505 74.295) (end 158.505 73.66) (width 0.25) (layer F.Cu) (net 5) (status 30))
 (segment (start 159.775 81.28) (end 161.29 79.765) (width 0.25) (layer F.Cu) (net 6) (status 20))
 (segment (start 154.305 81.28) (end 159.775 81.28) (width 0.25) (layer F.Cu) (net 6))
 (segment (start 146.685 80.01) (end 153.035 80.01) (width 0.25) (layer F.Cu) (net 6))
 (segment (start 145.415 73.72) (end 145.415 78.74) (width 0.25) (layer F.Cu) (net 6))
 (segment (start 153.035 80.01) (end 154.305 81.28) (width 0.25) (layer F.Cu) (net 6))
 (segment (start 145.415 78.74) (end 146.685 80.01) (width 0.25) (layer F.Cu) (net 6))
 (segment (start 147.955 74.055) (end 149.465 75.565) (width 0.25) (layer F.Cu) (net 7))
 (segment (start 147.955 73.72) (end 147.955 74.055) (width 0.25) (layer F.Cu) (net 7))
 (segment (start 149.465 75.565) (end 151.13 75.565) (width 0.25) (layer F.Cu) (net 7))
 (segment (start 155.33 79.765) (end 156.21 79.765) (width 0.25) (layer F.Cu) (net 7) (status 20))
 (segment (start 151.13 75.565) (end 155.33 79.765) (width 0.25) (layer F.Cu) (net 7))
 (segment (start 138.735 68.52) (end 138.43 68.825) (width 0.25) (layer F.Cu) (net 8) (status 30))
 (segment (start 139.31 66.86) (end 140.97 68.52) (width 0.25) (layer F.Cu) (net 8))
 (segment (start 139.31 60.96) (end 139.31 66.86) (width 0.25) (layer F.Cu) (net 8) (status 10))
 (segment (start 144.145 68.52) (end 140.97 68.52) (width 0.25) (layer F.Cu) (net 8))
 (segment (start 140.97 68.52) (end 138.735 68.52) (width 0.25) (layer F.Cu) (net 8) (status 20))
 (segment (start 153.425 68.58) (end 156.21 68.58) (width 0.25) (layer F.Cu) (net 9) (status 10))
 (segment (start 157.48 67.31) (end 160.02 67.31) (width 0.25) (layer F.Cu) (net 9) (status 20))
 (segment (start 156.21 68.58) (end 157.48 67.31) (width 0.25) (layer F.Cu) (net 9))
 (segment (start 146.685 76.59) (end 146.685 73.72) (width 0.25) (layer F.Cu) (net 10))
 (segment (start 147.565 77.47) (end 146.685 76.59) (width 0.25) (layer F.Cu) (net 10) (status 10))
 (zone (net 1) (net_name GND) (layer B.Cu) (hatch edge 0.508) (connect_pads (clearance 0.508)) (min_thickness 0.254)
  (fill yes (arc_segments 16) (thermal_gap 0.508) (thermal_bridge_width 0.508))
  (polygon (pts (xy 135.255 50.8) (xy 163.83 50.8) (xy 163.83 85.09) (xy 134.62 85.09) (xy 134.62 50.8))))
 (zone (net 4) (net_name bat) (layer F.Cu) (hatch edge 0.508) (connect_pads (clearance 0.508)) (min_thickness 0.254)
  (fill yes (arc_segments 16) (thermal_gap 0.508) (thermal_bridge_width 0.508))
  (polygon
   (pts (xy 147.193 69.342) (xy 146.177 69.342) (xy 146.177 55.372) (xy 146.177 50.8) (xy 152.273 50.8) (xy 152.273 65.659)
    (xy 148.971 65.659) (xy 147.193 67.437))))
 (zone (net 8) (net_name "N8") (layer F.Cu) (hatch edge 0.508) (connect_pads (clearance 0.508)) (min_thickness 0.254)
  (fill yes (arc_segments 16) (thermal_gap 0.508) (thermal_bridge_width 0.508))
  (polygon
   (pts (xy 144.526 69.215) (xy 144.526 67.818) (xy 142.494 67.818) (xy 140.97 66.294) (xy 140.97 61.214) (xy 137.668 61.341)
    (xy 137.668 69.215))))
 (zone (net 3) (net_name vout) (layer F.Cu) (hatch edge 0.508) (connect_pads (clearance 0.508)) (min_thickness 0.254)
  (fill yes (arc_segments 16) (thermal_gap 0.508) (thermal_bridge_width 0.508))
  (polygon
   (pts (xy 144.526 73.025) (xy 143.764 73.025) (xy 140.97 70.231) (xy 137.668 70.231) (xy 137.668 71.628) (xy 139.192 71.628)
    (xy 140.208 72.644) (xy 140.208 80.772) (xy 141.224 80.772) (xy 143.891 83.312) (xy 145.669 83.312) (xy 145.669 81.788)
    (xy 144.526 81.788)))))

